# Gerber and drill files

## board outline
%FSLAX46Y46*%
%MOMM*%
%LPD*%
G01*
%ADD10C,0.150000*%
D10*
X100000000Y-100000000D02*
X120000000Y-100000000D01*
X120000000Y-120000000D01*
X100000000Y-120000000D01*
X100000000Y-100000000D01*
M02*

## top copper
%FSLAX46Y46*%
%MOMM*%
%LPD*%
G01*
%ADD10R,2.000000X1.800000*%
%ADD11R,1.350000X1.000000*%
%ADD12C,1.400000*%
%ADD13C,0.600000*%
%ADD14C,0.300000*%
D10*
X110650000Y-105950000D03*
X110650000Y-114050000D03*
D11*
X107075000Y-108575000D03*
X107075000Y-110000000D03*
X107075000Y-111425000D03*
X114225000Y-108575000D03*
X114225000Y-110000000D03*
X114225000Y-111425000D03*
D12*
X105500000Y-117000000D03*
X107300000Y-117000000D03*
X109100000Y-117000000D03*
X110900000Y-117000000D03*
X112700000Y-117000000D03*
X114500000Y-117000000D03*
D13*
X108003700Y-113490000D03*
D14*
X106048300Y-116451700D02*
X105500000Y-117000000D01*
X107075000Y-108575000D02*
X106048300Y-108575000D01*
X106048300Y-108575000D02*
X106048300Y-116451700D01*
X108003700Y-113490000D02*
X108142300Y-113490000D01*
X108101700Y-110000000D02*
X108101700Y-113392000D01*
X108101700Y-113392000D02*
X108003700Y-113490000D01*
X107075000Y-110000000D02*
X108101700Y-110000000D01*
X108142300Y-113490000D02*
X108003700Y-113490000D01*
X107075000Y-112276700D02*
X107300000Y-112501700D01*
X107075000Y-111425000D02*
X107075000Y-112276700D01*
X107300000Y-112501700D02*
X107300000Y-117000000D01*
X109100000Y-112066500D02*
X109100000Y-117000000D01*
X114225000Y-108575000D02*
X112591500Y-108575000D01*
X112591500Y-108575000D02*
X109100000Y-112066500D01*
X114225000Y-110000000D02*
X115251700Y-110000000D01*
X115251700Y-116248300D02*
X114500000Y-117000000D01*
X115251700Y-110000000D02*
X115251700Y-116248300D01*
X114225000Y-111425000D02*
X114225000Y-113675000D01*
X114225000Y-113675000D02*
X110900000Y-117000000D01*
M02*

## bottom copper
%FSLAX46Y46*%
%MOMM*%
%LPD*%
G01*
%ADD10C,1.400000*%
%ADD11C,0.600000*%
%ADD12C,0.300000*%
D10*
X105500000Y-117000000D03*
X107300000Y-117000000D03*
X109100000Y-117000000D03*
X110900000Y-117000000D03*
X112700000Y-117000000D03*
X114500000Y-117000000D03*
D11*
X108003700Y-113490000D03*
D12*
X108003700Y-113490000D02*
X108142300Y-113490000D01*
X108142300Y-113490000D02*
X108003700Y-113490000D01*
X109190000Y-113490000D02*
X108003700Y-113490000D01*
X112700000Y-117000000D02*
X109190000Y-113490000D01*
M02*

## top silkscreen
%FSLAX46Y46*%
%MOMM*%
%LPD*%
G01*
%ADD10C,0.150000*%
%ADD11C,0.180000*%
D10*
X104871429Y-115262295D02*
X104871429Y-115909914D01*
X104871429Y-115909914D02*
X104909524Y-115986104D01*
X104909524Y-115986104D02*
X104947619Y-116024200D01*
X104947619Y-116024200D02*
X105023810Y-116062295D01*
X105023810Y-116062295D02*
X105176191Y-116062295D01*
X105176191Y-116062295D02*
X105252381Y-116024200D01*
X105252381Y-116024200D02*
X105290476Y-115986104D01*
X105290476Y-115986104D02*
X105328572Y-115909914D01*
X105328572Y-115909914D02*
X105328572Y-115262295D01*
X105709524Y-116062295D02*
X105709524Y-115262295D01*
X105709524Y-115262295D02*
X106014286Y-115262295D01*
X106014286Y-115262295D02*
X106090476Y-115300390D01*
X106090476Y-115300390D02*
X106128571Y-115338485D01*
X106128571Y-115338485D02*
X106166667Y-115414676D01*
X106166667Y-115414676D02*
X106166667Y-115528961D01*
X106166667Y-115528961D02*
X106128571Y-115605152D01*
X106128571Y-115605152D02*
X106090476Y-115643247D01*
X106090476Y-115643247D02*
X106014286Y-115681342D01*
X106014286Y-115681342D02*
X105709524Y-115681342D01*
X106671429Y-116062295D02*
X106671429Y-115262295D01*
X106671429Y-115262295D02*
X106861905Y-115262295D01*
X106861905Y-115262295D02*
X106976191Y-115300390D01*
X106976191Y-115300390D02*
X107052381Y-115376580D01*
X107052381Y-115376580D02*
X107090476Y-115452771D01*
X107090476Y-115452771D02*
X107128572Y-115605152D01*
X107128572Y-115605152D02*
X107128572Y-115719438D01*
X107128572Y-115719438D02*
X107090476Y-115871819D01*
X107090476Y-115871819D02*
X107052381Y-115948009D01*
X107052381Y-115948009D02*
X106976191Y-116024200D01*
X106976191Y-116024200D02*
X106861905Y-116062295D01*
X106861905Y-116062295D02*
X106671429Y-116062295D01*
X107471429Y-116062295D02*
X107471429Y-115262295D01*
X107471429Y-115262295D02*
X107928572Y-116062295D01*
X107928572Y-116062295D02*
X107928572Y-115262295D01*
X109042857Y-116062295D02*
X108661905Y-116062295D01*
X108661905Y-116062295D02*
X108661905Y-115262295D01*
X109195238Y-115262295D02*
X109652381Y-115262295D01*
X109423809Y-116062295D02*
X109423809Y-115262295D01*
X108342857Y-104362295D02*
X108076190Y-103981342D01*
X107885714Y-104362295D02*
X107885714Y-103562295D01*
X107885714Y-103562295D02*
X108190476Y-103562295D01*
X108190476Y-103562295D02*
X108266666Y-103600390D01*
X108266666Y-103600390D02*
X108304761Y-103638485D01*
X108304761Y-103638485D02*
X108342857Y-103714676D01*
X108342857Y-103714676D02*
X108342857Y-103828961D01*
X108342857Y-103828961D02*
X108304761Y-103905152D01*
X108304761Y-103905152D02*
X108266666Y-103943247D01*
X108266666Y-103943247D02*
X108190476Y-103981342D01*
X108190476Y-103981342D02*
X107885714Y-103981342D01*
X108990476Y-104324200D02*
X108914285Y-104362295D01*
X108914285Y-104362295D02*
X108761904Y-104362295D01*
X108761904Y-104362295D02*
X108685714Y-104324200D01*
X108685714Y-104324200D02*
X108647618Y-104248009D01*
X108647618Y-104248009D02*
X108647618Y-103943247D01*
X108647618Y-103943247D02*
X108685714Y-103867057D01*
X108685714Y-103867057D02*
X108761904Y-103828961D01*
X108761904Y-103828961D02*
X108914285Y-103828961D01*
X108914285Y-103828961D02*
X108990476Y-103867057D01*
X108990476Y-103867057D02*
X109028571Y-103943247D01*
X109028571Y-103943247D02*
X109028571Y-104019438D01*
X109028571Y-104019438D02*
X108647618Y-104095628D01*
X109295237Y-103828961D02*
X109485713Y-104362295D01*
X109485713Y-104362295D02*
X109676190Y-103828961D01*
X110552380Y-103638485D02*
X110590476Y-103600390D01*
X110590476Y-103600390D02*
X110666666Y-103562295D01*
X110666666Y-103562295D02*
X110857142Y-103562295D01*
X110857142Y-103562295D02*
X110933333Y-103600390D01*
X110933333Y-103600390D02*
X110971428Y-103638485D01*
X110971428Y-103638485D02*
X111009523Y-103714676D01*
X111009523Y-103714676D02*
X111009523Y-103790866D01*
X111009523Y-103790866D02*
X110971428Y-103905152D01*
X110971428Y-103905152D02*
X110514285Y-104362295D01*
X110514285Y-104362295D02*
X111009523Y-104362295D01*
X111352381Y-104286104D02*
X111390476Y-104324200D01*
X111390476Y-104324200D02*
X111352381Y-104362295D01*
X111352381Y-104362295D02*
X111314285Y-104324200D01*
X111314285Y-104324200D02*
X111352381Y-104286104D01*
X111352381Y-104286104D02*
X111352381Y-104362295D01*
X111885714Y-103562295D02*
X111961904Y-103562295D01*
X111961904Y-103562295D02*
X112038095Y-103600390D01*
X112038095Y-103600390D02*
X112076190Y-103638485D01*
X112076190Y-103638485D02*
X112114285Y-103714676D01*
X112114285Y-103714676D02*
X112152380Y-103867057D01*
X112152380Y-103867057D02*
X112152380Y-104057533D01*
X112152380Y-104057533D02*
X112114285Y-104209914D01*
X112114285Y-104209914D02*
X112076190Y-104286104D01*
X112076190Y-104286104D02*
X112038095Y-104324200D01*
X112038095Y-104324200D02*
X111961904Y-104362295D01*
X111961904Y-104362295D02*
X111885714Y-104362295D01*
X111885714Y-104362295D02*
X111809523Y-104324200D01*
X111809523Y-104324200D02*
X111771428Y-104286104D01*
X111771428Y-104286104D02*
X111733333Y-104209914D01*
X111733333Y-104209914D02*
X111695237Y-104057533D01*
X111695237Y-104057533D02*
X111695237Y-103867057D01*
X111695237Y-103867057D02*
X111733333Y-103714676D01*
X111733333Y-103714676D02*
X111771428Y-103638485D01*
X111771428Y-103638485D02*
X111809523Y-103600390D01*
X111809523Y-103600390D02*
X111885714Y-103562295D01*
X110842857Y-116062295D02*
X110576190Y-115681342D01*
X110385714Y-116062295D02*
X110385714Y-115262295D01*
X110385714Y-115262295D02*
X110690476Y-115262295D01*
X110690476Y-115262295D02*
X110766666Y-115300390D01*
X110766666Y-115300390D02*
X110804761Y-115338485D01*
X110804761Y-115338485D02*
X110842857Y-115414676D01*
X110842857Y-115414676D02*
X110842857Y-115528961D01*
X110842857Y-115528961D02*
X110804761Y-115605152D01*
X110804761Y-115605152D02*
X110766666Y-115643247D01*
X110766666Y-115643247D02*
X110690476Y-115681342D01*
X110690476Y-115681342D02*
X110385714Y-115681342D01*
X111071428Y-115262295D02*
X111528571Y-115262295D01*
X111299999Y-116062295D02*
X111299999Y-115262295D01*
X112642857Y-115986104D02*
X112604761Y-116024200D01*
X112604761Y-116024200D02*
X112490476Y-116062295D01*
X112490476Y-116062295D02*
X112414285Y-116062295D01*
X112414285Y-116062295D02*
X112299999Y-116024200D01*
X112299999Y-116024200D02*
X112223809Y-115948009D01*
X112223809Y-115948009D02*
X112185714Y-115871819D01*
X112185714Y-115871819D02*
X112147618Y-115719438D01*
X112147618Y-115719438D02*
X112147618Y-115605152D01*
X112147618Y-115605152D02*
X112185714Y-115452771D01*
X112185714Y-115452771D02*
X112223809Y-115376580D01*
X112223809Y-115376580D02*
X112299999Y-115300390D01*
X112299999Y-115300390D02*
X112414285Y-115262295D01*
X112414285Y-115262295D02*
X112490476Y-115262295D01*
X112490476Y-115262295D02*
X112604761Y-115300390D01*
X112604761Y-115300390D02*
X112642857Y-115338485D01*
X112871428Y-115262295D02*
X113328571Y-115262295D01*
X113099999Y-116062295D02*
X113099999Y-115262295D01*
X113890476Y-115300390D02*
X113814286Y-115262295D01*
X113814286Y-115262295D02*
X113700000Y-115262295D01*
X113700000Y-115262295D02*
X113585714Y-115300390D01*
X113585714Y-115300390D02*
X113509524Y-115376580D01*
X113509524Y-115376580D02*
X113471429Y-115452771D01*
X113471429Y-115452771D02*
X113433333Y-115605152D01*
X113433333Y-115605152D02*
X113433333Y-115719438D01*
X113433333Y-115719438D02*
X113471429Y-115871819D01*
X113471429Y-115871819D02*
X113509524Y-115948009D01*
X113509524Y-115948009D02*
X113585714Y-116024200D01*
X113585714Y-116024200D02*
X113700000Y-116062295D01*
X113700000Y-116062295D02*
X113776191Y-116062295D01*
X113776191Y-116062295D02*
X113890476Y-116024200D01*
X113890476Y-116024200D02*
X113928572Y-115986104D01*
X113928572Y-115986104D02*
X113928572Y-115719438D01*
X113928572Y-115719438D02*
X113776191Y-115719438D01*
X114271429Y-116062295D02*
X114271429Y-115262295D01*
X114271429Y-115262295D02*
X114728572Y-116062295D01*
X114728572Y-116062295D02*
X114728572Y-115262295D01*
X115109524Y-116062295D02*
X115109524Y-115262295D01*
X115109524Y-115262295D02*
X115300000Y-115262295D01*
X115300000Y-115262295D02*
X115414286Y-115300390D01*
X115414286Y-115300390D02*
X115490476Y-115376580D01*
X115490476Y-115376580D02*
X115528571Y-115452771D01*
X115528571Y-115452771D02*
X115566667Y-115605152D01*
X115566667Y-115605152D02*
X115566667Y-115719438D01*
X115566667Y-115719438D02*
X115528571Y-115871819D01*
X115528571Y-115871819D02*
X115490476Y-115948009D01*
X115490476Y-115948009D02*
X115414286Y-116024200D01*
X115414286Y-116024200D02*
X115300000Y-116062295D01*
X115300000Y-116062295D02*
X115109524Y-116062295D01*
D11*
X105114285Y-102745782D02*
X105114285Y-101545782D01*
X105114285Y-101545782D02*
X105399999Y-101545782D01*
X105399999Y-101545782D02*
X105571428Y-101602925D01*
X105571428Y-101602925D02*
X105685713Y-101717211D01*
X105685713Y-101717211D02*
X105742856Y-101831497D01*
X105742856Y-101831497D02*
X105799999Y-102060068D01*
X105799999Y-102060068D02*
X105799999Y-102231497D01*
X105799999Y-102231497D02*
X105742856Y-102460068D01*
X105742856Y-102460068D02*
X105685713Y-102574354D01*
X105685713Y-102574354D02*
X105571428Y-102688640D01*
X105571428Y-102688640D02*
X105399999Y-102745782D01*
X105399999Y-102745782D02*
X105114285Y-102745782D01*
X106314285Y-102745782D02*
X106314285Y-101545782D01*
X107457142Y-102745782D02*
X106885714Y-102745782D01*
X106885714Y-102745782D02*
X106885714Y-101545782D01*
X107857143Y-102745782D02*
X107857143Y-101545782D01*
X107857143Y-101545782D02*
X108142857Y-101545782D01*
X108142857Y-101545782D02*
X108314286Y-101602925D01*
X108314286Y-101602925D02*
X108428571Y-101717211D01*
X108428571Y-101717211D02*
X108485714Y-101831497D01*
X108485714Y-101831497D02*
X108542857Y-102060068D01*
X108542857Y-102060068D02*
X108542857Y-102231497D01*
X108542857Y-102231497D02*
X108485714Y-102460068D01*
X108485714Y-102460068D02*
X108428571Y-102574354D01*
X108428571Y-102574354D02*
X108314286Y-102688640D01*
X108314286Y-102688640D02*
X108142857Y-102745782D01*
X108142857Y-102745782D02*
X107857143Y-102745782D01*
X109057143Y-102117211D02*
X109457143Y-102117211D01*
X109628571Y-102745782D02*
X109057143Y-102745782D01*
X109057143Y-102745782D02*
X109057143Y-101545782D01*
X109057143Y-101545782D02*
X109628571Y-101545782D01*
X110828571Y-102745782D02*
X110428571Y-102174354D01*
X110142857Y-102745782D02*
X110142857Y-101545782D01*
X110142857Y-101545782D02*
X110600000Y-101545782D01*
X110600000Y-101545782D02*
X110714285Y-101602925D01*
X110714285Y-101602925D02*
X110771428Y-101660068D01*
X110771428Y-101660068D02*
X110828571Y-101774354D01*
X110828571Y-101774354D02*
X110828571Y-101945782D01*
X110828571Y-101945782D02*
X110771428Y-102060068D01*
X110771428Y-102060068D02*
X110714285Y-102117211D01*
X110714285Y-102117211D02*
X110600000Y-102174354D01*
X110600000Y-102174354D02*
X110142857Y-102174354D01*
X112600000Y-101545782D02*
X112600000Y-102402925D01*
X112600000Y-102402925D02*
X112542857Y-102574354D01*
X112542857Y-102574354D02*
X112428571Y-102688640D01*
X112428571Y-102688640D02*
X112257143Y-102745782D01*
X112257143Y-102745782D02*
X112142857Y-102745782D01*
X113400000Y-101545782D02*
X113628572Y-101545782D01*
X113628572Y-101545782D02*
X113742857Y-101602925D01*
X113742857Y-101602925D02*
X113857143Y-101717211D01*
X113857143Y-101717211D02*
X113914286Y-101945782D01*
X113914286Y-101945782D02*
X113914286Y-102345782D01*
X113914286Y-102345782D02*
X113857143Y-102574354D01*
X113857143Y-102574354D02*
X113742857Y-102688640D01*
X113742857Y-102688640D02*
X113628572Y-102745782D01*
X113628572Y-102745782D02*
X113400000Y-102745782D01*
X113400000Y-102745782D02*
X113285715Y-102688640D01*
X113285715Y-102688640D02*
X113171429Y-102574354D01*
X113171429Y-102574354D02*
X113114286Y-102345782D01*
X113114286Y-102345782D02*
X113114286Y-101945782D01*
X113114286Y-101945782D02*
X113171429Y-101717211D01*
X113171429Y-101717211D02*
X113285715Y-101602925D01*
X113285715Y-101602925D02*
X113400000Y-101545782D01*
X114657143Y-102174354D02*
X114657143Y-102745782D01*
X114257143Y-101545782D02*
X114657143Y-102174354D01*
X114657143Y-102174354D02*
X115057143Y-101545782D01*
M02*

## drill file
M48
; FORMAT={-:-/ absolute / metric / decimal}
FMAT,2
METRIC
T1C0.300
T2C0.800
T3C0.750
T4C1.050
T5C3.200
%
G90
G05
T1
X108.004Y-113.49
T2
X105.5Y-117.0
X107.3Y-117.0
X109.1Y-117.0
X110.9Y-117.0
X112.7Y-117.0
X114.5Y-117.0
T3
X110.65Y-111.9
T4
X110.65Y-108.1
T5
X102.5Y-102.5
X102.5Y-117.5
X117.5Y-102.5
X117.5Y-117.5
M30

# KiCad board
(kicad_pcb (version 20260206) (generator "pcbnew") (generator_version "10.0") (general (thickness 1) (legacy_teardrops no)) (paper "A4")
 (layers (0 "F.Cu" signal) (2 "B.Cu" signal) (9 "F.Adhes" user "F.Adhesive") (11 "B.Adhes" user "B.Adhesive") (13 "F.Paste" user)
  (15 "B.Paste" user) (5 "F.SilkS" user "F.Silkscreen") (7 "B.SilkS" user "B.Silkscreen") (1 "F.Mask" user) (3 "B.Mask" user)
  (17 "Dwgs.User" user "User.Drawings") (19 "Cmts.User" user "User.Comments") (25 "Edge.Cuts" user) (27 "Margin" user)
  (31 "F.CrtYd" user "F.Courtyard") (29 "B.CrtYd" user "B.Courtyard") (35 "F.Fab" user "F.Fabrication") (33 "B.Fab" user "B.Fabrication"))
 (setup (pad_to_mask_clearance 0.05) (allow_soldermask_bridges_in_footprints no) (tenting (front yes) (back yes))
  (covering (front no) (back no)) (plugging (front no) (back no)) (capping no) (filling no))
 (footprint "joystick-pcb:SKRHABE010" (layer "F.Cu") (at 110.65 110)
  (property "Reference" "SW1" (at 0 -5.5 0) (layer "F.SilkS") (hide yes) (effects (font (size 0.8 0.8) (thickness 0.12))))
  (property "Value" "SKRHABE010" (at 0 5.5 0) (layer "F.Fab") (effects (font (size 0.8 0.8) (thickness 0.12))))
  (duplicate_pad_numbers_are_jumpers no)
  (pad "" smd rect (at 0 -4.05) (size 2 1.8) (layers "F.Cu" "F.Mask" "F.Paste"))
  (pad "" np_thru_hole circle (at 0 -1.9) (size 1.05 1.05) (drill 1.05) (layers "*.Mask"))
  (pad "" np_thru_hole circle (at 0 1.9) (size 0.75 0.75) (drill 0.75) (layers "*.Mask"))
  (pad "" smd rect (at 0 4.05) (size 2 1.8) (layers "F.Cu" "F.Mask" "F.Paste"))
  (pad "1" smd rect (at -3.575 -1.425) (size 1.35 1) (layers "F.Cu" "F.Mask" "F.Paste") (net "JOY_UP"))
  (pad "2" smd rect (at -3.575 0) (size 1.35 1) (layers "F.Cu" "F.Mask" "F.Paste") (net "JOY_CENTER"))
  (pad "3" smd rect (at -3.575 1.425) (size 1.35 1) (layers "F.Cu" "F.Mask" "F.Paste") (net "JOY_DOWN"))
  (pad "4" smd rect (at 3.575 -1.425) (size 1.35 1) (layers "F.Cu" "F.Mask" "F.Paste") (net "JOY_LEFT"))
  (pad "5" smd rect (at 3.575 0) (size 1.35 1) (layers "F.Cu" "F.Mask" "F.Paste") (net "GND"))
  (pad "6" smd rect (at 3.575 1.425) (size 1.35 1) (layers "F.Cu" "F.Mask" "F.Paste") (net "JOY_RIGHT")))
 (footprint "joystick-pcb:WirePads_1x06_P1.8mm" (layer "F.Cu") (at 110 117)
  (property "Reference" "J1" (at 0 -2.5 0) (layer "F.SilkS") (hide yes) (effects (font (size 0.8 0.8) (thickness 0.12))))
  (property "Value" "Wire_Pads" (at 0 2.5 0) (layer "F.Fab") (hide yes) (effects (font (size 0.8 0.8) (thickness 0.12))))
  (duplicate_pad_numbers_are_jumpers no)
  (pad "1" thru_hole circle (at -4.5 0) (size 1.4 1.4) (drill 0.8) (layers "*.Cu" "*.Mask") (remove_unused_layers no) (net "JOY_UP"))
  (pad "2" thru_hole circle (at -2.7 0) (size 1.4 1.4) (drill 0.8) (layers "*.Cu" "*.Mask") (remove_unused_layers no) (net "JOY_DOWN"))
  (pad "3" thru_hole circle (at -0.9 0) (size 1.4 1.4) (drill 0.8) (layers "*.Cu" "*.Mask") (remove_unused_layers no) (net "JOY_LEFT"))
  (pad "4" thru_hole circle (at 0.9 0) (size 1.4 1.4) (drill 0.8) (layers "*.Cu" "*.Mask") (remove_unused_layers no) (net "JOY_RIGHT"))
  (pad "5" thru_hole circle (at 2.7 0) (size 1.4 1.4) (drill 0.8) (layers "*.Cu" "*.Mask") (remove_unused_layers no) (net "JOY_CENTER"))
  (pad "6" thru_hole circle (at 4.5 0) (size 1.4 1.4) (drill 0.8) (layers "*.Cu" "*.Mask") (remove_unused_layers no) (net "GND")))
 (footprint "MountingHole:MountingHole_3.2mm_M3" (layer "F.Cu") (at 102.5 102.5)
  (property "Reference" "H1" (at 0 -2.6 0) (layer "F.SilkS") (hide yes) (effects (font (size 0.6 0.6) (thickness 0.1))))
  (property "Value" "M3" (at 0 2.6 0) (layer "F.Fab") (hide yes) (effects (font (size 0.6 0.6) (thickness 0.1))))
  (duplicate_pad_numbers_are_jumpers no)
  (pad "" np_thru_hole circle (at 0 0) (size 3.2 3.2) (drill 3.2) (layers "*.Cu" "*.Mask")))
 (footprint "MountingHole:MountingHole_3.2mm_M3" (layer "F.Cu") (at 117.5 102.5)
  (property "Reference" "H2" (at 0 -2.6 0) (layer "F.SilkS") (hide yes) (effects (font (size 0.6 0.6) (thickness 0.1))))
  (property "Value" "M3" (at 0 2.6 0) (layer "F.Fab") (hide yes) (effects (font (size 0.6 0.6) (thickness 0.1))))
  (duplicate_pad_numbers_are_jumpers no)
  (pad "" np_thru_hole circle (at 0 0) (size 3.2 3.2) (drill 3.2) (layers "*.Cu" "*.Mask")))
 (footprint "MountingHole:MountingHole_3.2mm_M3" (layer "F.Cu") (at 102.5 117.5)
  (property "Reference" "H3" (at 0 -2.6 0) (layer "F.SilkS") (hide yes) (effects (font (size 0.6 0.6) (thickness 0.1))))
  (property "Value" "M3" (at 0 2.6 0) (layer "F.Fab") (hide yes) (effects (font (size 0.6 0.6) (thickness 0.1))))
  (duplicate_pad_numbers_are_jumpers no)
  (pad "" np_thru_hole circle (at 0 0) (size 3.2 3.2) (drill 3.2) (layers "*.Cu" "*.Mask")))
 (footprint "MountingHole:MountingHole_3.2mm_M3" (layer "F.Cu") (at 117.5 117.5)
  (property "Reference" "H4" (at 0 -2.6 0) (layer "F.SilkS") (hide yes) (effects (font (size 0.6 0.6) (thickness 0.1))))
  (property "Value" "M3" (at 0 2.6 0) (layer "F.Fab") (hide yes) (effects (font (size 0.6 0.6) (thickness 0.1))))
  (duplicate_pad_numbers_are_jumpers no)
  (pad "" np_thru_hole circle (at 0 0) (size 3.2 3.2) (drill 3.2) (layers "*.Cu" "*.Mask")))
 (gr_rect (start 100 100) (end 120 120) (stroke (width 0.15) (type default)) (fill no) (layer "Edge.Cuts"))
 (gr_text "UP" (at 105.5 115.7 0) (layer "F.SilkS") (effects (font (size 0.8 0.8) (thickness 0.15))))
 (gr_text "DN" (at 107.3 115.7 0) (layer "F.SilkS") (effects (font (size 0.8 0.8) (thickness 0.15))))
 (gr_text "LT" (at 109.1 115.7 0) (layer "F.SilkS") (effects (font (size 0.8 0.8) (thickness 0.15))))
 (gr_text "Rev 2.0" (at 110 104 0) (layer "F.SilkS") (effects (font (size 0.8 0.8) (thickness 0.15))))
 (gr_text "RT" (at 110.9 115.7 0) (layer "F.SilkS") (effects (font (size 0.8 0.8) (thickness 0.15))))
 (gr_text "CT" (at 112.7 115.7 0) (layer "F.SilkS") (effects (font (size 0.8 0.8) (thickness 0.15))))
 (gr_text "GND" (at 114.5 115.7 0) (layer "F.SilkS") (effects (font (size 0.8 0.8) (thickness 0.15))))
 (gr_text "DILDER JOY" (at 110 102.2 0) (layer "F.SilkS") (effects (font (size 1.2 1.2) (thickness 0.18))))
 (segment (start 106.0483 116.4517) (end 105.5 117) (width 0.3) (layer "F.Cu") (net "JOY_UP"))
 (segment (start 107.075 108.575) (end 106.0483 108.575) (width 0.3) (layer "F.Cu") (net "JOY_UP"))
 (segment (start 106.0483 108.575) (end 106.0483 116.4517) (width 0.3) (layer "F.Cu") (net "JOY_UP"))
 (segment (start 108.0037 113.49) (end 108.1423 113.49) (width 0.3) (layer "F.Cu") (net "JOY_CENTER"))
 (segment (start 108.1017 110) (end 108.1017 113.392) (width 0.3) (layer "F.Cu") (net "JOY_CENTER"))
 (segment (start 108.1017 113.392) (end 108.0037 113.49) (width 0.3) (layer "F.Cu") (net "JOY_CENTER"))
 (segment (start 107.075 110) (end 108.1017 110) (width 0.3) (layer "F.Cu") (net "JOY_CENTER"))
 (segment (start 108.1423 113.49) (end 108.0037 113.49) (width 0.3) (layer "F.Cu") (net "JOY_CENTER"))
 (via (at 108.0037 113.49) (size 0.6) (drill 0.3) (layers "F.Cu" "B.Cu") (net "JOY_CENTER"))
 (segment (start 108.0037 113.49) (end 108.1423 113.49) (width 0.3) (layer "B.Cu") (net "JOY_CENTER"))
 (segment (start 108.1423 113.49) (end 108.0037 113.49) (width 0.3) (layer "B.Cu") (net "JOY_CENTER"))
 (segment (start 109.19 113.49) (end 108.0037 113.49) (width 0.3) (layer "B.Cu") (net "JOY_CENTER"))
 (segment (start 112.7 117) (end 109.19 113.49) (width 0.3) (layer "B.Cu") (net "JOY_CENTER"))
 (segment (start 107.075 112.2767) (end 107.3 112.5017) (width 0.3) (layer "F.Cu") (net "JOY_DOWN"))
 (segment (start 107.075 111.425) (end 107.075 112.2767) (width 0.3) (layer "F.Cu") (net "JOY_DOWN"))
 (segment (start 107.3 112.5017) (end 107.3 117) (width 0.3) (layer "F.Cu") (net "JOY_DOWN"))
 (segment (start 109.1 112.0665) (end 109.1 117) (width 0.3) (layer "F.Cu") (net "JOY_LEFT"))
 (segment (start 114.225 108.575) (end 112.5915 108.575) (width 0.3) (layer "F.Cu") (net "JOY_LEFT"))
 (segment (start 112.5915 108.575) (end 109.1 112.0665) (width 0.3) (layer "F.Cu") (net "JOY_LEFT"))
 (segment (start 114.225 110) (end 115.2517 110) (width 0.3) (layer "F.Cu") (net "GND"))
 (segment (start 115.2517 116.2483) (end 114.5 117) (width 0.3) (layer "F.Cu") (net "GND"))
 (segment (start 115.2517 110) (end 115.2517 116.2483) (width 0.3) (layer "F.Cu") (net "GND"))
 (segment (start 114.225 111.425) (end 114.225 113.675) (width 0.3) (layer "F.Cu") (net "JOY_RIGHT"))
 (segment (start 114.225 113.675) (end 110.9 117) (width 0.3) (layer "F.Cu") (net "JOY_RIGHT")))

